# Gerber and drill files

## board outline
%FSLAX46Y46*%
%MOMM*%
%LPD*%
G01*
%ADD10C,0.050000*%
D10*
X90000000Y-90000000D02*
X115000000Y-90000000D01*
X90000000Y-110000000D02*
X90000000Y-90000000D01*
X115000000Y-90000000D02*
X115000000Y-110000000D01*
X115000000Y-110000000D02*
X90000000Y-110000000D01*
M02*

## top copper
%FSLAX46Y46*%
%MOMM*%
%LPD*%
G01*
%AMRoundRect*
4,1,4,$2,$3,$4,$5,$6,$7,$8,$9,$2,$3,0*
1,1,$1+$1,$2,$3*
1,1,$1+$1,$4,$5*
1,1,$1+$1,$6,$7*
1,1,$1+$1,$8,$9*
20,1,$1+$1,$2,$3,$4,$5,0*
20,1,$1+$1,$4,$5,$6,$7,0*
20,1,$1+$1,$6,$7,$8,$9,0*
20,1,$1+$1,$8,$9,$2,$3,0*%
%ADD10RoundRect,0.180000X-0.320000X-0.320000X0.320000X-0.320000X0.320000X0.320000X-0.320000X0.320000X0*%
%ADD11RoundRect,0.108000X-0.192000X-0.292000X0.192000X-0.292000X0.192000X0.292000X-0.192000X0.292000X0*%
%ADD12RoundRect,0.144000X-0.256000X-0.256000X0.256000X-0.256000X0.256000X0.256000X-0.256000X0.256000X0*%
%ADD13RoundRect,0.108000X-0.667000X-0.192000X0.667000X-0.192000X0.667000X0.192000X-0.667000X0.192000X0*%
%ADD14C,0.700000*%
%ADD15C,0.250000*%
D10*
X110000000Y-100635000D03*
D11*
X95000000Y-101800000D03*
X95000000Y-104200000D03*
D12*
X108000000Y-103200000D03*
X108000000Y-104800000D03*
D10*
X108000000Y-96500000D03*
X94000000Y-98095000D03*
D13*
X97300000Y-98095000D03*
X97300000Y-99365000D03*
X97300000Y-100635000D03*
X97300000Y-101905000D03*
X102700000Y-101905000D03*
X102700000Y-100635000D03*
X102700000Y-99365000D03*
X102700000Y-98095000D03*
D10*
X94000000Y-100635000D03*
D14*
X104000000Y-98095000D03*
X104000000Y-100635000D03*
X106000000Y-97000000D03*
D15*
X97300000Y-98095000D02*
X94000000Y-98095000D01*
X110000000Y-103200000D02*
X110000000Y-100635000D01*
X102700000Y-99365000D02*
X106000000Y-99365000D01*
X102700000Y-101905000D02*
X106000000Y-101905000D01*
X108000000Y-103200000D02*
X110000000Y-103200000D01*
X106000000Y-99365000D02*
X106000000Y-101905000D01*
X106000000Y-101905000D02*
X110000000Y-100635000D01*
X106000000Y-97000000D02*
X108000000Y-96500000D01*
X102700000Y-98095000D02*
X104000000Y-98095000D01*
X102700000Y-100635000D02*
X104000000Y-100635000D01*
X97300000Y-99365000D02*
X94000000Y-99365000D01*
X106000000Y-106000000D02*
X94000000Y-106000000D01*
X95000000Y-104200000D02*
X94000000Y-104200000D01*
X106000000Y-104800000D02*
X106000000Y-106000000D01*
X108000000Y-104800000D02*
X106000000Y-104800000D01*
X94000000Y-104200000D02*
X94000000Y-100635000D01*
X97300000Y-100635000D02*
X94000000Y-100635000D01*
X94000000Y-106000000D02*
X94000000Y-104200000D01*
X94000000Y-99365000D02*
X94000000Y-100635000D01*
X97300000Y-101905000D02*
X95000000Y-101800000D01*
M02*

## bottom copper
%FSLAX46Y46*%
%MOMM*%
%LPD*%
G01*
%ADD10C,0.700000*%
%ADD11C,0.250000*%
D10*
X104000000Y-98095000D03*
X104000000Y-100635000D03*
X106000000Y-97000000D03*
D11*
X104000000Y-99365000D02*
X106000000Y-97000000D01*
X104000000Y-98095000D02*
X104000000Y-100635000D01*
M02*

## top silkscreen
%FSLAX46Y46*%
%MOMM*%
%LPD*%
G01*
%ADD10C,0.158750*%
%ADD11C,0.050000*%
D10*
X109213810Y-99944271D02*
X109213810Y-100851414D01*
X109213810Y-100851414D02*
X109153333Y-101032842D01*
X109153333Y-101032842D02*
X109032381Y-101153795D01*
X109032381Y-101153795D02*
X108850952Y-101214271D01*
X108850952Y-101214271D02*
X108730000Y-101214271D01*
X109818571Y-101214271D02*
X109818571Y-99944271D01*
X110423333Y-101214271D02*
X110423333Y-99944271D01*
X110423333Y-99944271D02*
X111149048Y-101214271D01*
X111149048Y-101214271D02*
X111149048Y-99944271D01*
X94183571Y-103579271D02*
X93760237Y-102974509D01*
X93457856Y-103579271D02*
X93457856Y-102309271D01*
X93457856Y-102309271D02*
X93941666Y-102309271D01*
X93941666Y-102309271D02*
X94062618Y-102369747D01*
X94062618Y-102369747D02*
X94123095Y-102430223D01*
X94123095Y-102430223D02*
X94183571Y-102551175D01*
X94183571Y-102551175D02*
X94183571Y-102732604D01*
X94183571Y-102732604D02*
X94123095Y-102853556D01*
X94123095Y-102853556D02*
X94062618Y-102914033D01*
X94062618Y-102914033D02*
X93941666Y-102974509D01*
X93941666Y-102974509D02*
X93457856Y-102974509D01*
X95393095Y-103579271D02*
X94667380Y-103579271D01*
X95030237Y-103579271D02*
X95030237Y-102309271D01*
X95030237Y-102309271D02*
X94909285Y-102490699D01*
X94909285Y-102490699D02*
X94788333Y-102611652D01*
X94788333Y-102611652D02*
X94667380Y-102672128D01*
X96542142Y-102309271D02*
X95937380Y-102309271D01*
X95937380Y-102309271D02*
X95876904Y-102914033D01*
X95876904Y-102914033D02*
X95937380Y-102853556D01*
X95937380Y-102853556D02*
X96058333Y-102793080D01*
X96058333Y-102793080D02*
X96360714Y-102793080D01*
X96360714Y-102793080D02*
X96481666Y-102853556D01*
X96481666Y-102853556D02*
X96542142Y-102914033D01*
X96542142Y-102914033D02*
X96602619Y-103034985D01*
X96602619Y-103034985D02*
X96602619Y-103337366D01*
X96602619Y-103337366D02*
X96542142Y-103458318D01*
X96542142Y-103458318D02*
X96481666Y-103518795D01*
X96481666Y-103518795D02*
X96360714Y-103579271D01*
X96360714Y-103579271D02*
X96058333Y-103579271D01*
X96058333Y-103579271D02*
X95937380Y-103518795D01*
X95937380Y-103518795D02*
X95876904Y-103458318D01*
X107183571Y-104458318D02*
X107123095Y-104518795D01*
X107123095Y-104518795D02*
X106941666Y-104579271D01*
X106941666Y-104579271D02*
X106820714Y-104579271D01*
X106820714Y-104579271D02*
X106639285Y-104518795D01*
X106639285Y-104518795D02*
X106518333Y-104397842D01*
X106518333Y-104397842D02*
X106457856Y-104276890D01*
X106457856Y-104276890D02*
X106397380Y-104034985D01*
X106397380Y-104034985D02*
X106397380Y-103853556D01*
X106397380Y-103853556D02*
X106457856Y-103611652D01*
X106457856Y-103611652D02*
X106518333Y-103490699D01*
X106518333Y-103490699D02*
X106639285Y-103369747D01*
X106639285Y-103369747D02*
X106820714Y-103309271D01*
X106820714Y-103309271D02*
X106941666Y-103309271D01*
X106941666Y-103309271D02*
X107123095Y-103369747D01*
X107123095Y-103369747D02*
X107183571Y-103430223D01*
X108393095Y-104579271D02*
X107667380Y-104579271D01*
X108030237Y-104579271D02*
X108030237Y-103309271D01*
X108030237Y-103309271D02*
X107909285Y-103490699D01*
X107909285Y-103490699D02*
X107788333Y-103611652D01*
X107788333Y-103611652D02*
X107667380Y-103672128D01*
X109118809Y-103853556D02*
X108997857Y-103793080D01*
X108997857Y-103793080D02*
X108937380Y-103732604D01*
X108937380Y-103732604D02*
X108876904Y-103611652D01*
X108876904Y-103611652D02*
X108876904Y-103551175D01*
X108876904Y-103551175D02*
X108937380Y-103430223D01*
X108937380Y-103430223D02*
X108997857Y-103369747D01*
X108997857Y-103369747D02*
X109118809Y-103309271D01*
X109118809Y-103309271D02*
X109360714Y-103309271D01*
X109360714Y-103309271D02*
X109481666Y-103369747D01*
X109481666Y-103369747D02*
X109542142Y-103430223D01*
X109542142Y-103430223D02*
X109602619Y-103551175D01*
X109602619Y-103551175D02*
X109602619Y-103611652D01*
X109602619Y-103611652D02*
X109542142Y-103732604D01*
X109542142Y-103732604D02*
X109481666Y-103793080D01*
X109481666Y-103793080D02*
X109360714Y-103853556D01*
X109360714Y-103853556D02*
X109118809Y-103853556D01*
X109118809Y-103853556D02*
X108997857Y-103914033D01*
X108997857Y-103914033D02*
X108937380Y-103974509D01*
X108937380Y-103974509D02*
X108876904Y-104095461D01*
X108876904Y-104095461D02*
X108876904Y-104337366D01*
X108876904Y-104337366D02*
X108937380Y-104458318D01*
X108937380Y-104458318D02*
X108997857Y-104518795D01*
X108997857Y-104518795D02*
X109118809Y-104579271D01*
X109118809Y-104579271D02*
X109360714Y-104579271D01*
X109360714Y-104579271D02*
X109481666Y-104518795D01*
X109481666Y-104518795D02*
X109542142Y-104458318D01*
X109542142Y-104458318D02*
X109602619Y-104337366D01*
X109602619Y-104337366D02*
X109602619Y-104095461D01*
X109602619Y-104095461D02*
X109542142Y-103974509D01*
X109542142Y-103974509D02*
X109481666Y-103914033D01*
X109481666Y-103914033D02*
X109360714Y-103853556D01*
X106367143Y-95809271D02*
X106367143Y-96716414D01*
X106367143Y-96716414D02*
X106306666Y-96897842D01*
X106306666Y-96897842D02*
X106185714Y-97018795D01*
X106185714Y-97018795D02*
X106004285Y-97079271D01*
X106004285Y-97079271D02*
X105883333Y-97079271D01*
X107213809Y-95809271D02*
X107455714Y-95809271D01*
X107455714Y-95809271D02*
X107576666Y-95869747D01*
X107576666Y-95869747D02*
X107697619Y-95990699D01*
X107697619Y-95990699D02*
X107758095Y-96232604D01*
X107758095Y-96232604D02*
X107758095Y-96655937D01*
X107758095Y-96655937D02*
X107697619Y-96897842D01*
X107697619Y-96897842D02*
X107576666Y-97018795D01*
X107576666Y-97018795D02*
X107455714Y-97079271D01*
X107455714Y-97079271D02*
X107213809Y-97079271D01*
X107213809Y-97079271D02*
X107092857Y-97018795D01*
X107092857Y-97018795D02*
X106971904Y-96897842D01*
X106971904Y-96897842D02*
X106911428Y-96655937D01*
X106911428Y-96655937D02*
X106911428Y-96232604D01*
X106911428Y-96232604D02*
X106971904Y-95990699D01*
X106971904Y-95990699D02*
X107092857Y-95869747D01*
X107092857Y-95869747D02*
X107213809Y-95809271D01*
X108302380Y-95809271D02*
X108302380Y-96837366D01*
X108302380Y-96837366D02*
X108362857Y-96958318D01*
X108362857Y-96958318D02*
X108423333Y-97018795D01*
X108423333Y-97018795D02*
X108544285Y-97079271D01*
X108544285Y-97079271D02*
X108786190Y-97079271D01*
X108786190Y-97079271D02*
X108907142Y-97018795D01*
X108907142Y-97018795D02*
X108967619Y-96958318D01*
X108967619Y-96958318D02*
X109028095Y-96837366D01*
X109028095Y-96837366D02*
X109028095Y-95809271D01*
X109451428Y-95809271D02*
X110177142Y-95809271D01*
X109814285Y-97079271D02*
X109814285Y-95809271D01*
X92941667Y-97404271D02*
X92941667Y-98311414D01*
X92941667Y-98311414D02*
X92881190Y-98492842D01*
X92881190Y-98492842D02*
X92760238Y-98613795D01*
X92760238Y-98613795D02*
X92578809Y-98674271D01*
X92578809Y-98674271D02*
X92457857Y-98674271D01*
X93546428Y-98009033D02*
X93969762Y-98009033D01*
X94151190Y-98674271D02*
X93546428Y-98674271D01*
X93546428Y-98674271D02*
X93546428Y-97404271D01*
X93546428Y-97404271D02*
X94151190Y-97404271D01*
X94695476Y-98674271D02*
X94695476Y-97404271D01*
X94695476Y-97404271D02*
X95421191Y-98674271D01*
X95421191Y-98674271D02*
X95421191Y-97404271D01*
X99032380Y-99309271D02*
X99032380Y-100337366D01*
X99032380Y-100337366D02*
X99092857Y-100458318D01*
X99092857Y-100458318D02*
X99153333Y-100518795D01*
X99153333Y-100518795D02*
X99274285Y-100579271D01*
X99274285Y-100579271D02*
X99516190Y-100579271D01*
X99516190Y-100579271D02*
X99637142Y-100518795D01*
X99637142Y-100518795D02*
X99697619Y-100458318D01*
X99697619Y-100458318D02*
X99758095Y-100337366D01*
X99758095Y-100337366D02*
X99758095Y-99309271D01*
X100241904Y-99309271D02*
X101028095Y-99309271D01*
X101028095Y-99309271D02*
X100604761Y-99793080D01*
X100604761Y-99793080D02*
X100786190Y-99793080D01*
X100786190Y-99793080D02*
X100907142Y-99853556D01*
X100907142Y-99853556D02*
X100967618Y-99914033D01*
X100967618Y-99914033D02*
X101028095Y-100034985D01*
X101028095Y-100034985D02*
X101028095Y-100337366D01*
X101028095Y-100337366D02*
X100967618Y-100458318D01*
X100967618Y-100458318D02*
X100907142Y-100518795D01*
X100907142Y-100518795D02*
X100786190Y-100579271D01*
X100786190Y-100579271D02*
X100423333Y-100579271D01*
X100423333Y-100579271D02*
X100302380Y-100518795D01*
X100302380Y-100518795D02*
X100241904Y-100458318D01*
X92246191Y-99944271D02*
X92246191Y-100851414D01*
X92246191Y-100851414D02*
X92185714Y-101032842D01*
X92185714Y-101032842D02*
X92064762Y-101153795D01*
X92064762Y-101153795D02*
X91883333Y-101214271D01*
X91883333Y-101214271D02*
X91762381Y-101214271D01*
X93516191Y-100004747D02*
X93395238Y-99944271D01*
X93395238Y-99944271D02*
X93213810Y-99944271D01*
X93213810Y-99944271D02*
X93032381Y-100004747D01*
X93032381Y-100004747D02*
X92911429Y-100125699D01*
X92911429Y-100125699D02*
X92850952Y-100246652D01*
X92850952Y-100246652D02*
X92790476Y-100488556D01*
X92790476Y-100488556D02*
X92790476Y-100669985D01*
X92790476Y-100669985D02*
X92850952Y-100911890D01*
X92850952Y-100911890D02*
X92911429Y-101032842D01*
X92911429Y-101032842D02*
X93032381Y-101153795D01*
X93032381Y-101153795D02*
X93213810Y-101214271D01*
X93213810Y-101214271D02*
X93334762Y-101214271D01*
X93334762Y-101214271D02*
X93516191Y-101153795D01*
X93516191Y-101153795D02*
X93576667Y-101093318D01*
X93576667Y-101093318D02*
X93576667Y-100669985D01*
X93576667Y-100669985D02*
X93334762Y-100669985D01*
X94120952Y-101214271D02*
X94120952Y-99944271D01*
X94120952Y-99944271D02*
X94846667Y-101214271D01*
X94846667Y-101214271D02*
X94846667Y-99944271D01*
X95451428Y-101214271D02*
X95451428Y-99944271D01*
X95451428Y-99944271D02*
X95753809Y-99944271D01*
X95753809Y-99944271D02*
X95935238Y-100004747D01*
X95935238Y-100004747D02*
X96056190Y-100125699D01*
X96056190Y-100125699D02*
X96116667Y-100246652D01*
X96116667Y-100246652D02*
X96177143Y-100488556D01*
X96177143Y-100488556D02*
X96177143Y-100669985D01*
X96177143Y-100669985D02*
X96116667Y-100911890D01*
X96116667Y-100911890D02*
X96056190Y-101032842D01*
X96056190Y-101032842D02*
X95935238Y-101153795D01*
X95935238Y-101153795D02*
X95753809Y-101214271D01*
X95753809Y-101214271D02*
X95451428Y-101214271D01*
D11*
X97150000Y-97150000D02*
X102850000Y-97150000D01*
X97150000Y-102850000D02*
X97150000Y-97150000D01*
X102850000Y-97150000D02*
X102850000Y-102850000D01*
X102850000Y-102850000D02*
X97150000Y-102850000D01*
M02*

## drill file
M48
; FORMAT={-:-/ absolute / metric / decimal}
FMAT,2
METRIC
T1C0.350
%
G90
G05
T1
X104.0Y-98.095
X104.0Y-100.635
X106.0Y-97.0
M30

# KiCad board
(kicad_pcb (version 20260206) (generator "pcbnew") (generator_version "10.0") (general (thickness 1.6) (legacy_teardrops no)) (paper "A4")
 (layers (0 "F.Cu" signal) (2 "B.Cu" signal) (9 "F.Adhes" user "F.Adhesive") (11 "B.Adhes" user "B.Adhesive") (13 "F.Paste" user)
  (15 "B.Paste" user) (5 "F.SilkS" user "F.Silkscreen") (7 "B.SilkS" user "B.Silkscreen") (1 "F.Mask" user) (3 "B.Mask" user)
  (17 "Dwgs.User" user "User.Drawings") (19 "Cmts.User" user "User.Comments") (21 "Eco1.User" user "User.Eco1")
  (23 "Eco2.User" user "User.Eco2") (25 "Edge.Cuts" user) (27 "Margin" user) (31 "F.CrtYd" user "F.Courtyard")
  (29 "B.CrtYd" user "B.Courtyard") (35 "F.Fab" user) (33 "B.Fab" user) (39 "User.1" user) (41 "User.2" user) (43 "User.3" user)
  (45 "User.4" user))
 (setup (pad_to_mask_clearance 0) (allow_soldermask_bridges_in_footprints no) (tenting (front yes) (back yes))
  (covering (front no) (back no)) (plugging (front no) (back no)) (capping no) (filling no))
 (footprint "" (layer "F.Cu") (at 110 100.635)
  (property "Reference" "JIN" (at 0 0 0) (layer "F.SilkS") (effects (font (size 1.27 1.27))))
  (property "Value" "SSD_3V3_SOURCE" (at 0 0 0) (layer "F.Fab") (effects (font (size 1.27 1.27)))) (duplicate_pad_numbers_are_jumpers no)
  (pad "1" smd roundrect (at 0 0) (size 1 1) (layers "F.Cu") (roundrect_rratio 0.18) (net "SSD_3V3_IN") (solder_mask_margin 0)
   (solder_paste_margin -0.05) (solder_paste_margin_ratio 0) (thermal_bridge_angle 45)))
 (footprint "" (layer "F.Cu") (at 95 103)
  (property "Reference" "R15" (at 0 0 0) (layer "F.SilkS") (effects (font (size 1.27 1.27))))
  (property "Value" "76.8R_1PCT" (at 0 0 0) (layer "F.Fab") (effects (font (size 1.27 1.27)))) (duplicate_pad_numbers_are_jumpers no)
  (pad "1" smd roundrect (at 0 -1.2) (size 0.6 0.8) (layers "F.Cu") (roundrect_rratio 0.18) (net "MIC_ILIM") (solder_mask_margin 0)
   (solder_paste_margin -0.05) (solder_paste_margin_ratio 0) (thermal_bridge_angle 45))
  (pad "2" smd roundrect (at 0 1.2) (size 0.6 0.8) (layers "F.Cu") (roundrect_rratio 0.18) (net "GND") (solder_mask_margin 0)
   (solder_paste_margin -0.05) (solder_paste_margin_ratio 0) (thermal_bridge_angle 45)))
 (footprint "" (layer "F.Cu") (at 108 104)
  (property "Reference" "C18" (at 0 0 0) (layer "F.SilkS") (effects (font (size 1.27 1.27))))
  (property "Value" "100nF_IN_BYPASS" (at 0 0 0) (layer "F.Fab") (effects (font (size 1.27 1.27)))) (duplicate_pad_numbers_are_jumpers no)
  (pad "1" smd roundrect (at 0 -0.8) (size 0.8 0.8) (layers "F.Cu") (roundrect_rratio 0.18) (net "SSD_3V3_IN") (solder_mask_margin 0)
   (solder_paste_margin -0.05) (solder_paste_margin_ratio 0) (thermal_bridge_angle 45))
  (pad "2" smd roundrect (at 0 0.8) (size 0.8 0.8) (layers "F.Cu") (roundrect_rratio 0.18) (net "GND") (solder_mask_margin 0)
   (solder_paste_margin -0.05) (solder_paste_margin_ratio 0) (thermal_bridge_angle 45)))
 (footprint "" (layer "F.Cu") (at 108 96.5)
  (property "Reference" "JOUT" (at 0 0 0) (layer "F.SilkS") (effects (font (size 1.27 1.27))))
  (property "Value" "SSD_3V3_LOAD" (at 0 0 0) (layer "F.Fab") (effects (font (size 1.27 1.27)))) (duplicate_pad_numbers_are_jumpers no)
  (pad "1" smd roundrect (at 0 0) (size 1 1) (layers "F.Cu") (roundrect_rratio 0.18) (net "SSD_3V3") (solder_mask_margin 0)
   (solder_paste_margin -0.05) (solder_paste_margin_ratio 0) (thermal_bridge_angle 45)))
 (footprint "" (layer "F.Cu") (at 94 98.095)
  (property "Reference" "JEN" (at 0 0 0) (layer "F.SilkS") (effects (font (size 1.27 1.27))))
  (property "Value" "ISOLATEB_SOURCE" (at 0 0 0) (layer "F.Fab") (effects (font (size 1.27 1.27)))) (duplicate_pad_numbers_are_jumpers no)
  (pad "1" smd roundrect (at 0 0) (size 1 1) (layers "F.Cu") (roundrect_rratio 0.18) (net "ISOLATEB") (solder_mask_margin 0)
   (solder_paste_margin -0.05) (solder_paste_margin_ratio 0) (thermal_bridge_angle 45)))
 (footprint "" (layer "F.Cu") (at 100 100)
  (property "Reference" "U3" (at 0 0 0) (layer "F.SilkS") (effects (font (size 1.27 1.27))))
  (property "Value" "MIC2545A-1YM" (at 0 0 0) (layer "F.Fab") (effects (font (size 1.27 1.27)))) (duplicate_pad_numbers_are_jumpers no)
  (fp_line (start -2.85 -2.85) (end 2.85 -2.85) (stroke (width 0.05) (type default)) (layer "F.SilkS"))
  (fp_line (start -2.85 2.85) (end -2.85 -2.85) (stroke (width 0.05) (type default)) (layer "F.SilkS"))
  (fp_line (start 2.85 -2.85) (end 2.85 2.85) (stroke (width 0.05) (type default)) (layer "F.SilkS"))
  (fp_line (start 2.85 2.85) (end -2.85 2.85) (stroke (width 0.05) (type default)) (layer "F.SilkS"))
  (pad "1" smd roundrect (at -2.7 -1.905) (size 1.55 0.6) (layers "F.Cu") (roundrect_rratio 0.18) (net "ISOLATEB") (solder_mask_margin 0)
   (solder_paste_margin -0.05) (solder_paste_margin_ratio 0) (thermal_bridge_angle 45))
  (pad "2" smd roundrect (at -2.7 -0.635) (size 1.55 0.6) (layers "F.Cu") (roundrect_rratio 0.18) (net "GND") (solder_mask_margin 0)
   (solder_paste_margin -0.05) (solder_paste_margin_ratio 0) (thermal_bridge_angle 45))
  (pad "3" smd roundrect (at -2.7 0.635) (size 1.55 0.6) (layers "F.Cu") (roundrect_rratio 0.18) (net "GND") (solder_mask_margin 0)
   (solder_paste_margin -0.05) (solder_paste_margin_ratio 0) (thermal_bridge_angle 45))
  (pad "4" smd roundrect (at -2.7 1.905) (size 1.55 0.6) (layers "F.Cu") (roundrect_rratio 0.18) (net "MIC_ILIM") (solder_mask_margin 0)
   (solder_paste_margin -0.05) (solder_paste_margin_ratio 0) (thermal_bridge_angle 45))
  (pad "5" smd roundrect (at 2.7 1.905) (size 1.55 0.6) (layers "F.Cu") (roundrect_rratio 0.18) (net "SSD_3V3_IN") (solder_mask_margin 0)
   (solder_paste_margin -0.05) (solder_paste_margin_ratio 0) (thermal_bridge_angle 45))
  (pad "6" smd roundrect (at 2.7 0.635) (size 1.55 0.6) (layers "F.Cu") (roundrect_rratio 0.18) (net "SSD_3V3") (solder_mask_margin 0)
   (solder_paste_margin -0.05) (solder_paste_margin_ratio 0) (thermal_bridge_angle 45))
  (pad "7" smd roundrect (at 2.7 -0.635) (size 1.55 0.6) (layers "F.Cu") (roundrect_rratio 0.18) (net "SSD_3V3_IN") (solder_mask_margin 0)
   (solder_paste_margin -0.05) (solder_paste_margin_ratio 0) (thermal_bridge_angle 45))
  (pad "8" smd roundrect (at 2.7 -1.905) (size 1.55 0.6) (layers "F.Cu") (roundrect_rratio 0.18) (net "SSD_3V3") (solder_mask_margin 0)
   (solder_paste_margin -0.05) (solder_paste_margin_ratio 0) (thermal_bridge_angle 45)))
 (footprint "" (layer "F.Cu") (at 94 100.635)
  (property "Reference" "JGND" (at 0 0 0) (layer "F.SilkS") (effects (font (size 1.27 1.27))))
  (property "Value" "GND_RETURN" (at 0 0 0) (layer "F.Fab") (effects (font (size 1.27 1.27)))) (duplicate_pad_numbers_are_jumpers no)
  (pad "1" smd roundrect (at 0 0) (size 1 1) (layers "F.Cu") (roundrect_rratio 0.18) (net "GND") (solder_mask_margin 0)
   (solder_paste_margin -0.05) (solder_paste_margin_ratio 0) (thermal_bridge_angle 45)))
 (gr_line (start 90 90) (end 115 90) (stroke (width 0.05) (type default)) (layer "Edge.Cuts"))
 (gr_line (start 90 110) (end 90 90) (stroke (width 0.05) (type default)) (layer "Edge.Cuts"))
 (gr_line (start 115 90) (end 115 110) (stroke (width 0.05) (type default)) (layer "Edge.Cuts"))
 (gr_line (start 115 110) (end 90 110) (stroke (width 0.05) (type default)) (layer "Edge.Cuts"))
 (segment (start 97.3 98.095) (end 94 98.095) (width 0.25) (layer "F.Cu") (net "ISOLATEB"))
 (segment (start 110 103.2) (end 110 100.635) (width 0.25) (layer "F.Cu") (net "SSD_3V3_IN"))
 (segment (start 102.7 99.365) (end 106 99.365) (width 0.25) (layer "F.Cu") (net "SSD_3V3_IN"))
 (segment (start 102.7 101.905) (end 106 101.905) (width 0.25) (layer "F.Cu") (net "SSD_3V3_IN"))
 (segment (start 108 103.2) (end 110 103.2) (width 0.25) (layer "F.Cu") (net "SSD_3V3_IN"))
 (segment (start 106 99.365) (end 106 101.905) (width 0.25) (layer "F.Cu") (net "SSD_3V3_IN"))
 (segment (start 106 101.905) (end 110 100.635) (width 0.25) (layer "F.Cu") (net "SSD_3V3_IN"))
 (segment (start 106 97) (end 108 96.5) (width 0.25) (layer "F.Cu") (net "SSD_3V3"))
 (segment (start 102.7 98.095) (end 104 98.095) (width 0.25) (layer "F.Cu") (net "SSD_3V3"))
 (segment (start 102.7 100.635) (end 104 100.635) (width 0.25) (layer "F.Cu") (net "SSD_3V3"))
 (via (at 104 98.095) (size 0.7) (drill 0.35) (layers "F.Cu" "B.Cu") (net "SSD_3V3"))
 (via (at 104 100.635) (size 0.7) (drill 0.35) (layers "F.Cu" "B.Cu") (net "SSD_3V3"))
 (via (at 106 97) (size 0.7) (drill 0.35) (layers "F.Cu" "B.Cu") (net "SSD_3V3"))
 (segment (start 104 99.365) (end 106 97) (width 0.25) (layer "B.Cu") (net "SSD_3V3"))
 (segment (start 104 98.095) (end 104 100.635) (width 0.25) (layer "B.Cu") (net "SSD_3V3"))
 (segment (start 97.3 99.365) (end 94 99.365) (width 0.25) (layer "F.Cu") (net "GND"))
 (segment (start 106 106) (end 94 106) (width 0.25) (layer "F.Cu") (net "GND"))
 (segment (start 95 104.2) (end 94 104.2) (width 0.25) (layer "F.Cu") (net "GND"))
 (segment (start 106 104.8) (end 106 106) (width 0.25) (layer "F.Cu") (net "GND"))
 (segment (start 108 104.8) (end 106 104.8) (width 0.25) (layer "F.Cu") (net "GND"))
 (segment (start 94 104.2) (end 94 100.635) (width 0.25) (layer "F.Cu") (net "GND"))
 (segment (start 97.3 100.635) (end 94 100.635) (width 0.25) (layer "F.Cu") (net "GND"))
 (segment (start 94 106) (end 94 104.2) (width 0.25) (layer "F.Cu") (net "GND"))
 (segment (start 94 99.365) (end 94 100.635) (width 0.25) (layer "F.Cu") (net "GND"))
 (segment (start 97.3 101.905) (end 95 101.8) (width 0.25) (layer "F.Cu") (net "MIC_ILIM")))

